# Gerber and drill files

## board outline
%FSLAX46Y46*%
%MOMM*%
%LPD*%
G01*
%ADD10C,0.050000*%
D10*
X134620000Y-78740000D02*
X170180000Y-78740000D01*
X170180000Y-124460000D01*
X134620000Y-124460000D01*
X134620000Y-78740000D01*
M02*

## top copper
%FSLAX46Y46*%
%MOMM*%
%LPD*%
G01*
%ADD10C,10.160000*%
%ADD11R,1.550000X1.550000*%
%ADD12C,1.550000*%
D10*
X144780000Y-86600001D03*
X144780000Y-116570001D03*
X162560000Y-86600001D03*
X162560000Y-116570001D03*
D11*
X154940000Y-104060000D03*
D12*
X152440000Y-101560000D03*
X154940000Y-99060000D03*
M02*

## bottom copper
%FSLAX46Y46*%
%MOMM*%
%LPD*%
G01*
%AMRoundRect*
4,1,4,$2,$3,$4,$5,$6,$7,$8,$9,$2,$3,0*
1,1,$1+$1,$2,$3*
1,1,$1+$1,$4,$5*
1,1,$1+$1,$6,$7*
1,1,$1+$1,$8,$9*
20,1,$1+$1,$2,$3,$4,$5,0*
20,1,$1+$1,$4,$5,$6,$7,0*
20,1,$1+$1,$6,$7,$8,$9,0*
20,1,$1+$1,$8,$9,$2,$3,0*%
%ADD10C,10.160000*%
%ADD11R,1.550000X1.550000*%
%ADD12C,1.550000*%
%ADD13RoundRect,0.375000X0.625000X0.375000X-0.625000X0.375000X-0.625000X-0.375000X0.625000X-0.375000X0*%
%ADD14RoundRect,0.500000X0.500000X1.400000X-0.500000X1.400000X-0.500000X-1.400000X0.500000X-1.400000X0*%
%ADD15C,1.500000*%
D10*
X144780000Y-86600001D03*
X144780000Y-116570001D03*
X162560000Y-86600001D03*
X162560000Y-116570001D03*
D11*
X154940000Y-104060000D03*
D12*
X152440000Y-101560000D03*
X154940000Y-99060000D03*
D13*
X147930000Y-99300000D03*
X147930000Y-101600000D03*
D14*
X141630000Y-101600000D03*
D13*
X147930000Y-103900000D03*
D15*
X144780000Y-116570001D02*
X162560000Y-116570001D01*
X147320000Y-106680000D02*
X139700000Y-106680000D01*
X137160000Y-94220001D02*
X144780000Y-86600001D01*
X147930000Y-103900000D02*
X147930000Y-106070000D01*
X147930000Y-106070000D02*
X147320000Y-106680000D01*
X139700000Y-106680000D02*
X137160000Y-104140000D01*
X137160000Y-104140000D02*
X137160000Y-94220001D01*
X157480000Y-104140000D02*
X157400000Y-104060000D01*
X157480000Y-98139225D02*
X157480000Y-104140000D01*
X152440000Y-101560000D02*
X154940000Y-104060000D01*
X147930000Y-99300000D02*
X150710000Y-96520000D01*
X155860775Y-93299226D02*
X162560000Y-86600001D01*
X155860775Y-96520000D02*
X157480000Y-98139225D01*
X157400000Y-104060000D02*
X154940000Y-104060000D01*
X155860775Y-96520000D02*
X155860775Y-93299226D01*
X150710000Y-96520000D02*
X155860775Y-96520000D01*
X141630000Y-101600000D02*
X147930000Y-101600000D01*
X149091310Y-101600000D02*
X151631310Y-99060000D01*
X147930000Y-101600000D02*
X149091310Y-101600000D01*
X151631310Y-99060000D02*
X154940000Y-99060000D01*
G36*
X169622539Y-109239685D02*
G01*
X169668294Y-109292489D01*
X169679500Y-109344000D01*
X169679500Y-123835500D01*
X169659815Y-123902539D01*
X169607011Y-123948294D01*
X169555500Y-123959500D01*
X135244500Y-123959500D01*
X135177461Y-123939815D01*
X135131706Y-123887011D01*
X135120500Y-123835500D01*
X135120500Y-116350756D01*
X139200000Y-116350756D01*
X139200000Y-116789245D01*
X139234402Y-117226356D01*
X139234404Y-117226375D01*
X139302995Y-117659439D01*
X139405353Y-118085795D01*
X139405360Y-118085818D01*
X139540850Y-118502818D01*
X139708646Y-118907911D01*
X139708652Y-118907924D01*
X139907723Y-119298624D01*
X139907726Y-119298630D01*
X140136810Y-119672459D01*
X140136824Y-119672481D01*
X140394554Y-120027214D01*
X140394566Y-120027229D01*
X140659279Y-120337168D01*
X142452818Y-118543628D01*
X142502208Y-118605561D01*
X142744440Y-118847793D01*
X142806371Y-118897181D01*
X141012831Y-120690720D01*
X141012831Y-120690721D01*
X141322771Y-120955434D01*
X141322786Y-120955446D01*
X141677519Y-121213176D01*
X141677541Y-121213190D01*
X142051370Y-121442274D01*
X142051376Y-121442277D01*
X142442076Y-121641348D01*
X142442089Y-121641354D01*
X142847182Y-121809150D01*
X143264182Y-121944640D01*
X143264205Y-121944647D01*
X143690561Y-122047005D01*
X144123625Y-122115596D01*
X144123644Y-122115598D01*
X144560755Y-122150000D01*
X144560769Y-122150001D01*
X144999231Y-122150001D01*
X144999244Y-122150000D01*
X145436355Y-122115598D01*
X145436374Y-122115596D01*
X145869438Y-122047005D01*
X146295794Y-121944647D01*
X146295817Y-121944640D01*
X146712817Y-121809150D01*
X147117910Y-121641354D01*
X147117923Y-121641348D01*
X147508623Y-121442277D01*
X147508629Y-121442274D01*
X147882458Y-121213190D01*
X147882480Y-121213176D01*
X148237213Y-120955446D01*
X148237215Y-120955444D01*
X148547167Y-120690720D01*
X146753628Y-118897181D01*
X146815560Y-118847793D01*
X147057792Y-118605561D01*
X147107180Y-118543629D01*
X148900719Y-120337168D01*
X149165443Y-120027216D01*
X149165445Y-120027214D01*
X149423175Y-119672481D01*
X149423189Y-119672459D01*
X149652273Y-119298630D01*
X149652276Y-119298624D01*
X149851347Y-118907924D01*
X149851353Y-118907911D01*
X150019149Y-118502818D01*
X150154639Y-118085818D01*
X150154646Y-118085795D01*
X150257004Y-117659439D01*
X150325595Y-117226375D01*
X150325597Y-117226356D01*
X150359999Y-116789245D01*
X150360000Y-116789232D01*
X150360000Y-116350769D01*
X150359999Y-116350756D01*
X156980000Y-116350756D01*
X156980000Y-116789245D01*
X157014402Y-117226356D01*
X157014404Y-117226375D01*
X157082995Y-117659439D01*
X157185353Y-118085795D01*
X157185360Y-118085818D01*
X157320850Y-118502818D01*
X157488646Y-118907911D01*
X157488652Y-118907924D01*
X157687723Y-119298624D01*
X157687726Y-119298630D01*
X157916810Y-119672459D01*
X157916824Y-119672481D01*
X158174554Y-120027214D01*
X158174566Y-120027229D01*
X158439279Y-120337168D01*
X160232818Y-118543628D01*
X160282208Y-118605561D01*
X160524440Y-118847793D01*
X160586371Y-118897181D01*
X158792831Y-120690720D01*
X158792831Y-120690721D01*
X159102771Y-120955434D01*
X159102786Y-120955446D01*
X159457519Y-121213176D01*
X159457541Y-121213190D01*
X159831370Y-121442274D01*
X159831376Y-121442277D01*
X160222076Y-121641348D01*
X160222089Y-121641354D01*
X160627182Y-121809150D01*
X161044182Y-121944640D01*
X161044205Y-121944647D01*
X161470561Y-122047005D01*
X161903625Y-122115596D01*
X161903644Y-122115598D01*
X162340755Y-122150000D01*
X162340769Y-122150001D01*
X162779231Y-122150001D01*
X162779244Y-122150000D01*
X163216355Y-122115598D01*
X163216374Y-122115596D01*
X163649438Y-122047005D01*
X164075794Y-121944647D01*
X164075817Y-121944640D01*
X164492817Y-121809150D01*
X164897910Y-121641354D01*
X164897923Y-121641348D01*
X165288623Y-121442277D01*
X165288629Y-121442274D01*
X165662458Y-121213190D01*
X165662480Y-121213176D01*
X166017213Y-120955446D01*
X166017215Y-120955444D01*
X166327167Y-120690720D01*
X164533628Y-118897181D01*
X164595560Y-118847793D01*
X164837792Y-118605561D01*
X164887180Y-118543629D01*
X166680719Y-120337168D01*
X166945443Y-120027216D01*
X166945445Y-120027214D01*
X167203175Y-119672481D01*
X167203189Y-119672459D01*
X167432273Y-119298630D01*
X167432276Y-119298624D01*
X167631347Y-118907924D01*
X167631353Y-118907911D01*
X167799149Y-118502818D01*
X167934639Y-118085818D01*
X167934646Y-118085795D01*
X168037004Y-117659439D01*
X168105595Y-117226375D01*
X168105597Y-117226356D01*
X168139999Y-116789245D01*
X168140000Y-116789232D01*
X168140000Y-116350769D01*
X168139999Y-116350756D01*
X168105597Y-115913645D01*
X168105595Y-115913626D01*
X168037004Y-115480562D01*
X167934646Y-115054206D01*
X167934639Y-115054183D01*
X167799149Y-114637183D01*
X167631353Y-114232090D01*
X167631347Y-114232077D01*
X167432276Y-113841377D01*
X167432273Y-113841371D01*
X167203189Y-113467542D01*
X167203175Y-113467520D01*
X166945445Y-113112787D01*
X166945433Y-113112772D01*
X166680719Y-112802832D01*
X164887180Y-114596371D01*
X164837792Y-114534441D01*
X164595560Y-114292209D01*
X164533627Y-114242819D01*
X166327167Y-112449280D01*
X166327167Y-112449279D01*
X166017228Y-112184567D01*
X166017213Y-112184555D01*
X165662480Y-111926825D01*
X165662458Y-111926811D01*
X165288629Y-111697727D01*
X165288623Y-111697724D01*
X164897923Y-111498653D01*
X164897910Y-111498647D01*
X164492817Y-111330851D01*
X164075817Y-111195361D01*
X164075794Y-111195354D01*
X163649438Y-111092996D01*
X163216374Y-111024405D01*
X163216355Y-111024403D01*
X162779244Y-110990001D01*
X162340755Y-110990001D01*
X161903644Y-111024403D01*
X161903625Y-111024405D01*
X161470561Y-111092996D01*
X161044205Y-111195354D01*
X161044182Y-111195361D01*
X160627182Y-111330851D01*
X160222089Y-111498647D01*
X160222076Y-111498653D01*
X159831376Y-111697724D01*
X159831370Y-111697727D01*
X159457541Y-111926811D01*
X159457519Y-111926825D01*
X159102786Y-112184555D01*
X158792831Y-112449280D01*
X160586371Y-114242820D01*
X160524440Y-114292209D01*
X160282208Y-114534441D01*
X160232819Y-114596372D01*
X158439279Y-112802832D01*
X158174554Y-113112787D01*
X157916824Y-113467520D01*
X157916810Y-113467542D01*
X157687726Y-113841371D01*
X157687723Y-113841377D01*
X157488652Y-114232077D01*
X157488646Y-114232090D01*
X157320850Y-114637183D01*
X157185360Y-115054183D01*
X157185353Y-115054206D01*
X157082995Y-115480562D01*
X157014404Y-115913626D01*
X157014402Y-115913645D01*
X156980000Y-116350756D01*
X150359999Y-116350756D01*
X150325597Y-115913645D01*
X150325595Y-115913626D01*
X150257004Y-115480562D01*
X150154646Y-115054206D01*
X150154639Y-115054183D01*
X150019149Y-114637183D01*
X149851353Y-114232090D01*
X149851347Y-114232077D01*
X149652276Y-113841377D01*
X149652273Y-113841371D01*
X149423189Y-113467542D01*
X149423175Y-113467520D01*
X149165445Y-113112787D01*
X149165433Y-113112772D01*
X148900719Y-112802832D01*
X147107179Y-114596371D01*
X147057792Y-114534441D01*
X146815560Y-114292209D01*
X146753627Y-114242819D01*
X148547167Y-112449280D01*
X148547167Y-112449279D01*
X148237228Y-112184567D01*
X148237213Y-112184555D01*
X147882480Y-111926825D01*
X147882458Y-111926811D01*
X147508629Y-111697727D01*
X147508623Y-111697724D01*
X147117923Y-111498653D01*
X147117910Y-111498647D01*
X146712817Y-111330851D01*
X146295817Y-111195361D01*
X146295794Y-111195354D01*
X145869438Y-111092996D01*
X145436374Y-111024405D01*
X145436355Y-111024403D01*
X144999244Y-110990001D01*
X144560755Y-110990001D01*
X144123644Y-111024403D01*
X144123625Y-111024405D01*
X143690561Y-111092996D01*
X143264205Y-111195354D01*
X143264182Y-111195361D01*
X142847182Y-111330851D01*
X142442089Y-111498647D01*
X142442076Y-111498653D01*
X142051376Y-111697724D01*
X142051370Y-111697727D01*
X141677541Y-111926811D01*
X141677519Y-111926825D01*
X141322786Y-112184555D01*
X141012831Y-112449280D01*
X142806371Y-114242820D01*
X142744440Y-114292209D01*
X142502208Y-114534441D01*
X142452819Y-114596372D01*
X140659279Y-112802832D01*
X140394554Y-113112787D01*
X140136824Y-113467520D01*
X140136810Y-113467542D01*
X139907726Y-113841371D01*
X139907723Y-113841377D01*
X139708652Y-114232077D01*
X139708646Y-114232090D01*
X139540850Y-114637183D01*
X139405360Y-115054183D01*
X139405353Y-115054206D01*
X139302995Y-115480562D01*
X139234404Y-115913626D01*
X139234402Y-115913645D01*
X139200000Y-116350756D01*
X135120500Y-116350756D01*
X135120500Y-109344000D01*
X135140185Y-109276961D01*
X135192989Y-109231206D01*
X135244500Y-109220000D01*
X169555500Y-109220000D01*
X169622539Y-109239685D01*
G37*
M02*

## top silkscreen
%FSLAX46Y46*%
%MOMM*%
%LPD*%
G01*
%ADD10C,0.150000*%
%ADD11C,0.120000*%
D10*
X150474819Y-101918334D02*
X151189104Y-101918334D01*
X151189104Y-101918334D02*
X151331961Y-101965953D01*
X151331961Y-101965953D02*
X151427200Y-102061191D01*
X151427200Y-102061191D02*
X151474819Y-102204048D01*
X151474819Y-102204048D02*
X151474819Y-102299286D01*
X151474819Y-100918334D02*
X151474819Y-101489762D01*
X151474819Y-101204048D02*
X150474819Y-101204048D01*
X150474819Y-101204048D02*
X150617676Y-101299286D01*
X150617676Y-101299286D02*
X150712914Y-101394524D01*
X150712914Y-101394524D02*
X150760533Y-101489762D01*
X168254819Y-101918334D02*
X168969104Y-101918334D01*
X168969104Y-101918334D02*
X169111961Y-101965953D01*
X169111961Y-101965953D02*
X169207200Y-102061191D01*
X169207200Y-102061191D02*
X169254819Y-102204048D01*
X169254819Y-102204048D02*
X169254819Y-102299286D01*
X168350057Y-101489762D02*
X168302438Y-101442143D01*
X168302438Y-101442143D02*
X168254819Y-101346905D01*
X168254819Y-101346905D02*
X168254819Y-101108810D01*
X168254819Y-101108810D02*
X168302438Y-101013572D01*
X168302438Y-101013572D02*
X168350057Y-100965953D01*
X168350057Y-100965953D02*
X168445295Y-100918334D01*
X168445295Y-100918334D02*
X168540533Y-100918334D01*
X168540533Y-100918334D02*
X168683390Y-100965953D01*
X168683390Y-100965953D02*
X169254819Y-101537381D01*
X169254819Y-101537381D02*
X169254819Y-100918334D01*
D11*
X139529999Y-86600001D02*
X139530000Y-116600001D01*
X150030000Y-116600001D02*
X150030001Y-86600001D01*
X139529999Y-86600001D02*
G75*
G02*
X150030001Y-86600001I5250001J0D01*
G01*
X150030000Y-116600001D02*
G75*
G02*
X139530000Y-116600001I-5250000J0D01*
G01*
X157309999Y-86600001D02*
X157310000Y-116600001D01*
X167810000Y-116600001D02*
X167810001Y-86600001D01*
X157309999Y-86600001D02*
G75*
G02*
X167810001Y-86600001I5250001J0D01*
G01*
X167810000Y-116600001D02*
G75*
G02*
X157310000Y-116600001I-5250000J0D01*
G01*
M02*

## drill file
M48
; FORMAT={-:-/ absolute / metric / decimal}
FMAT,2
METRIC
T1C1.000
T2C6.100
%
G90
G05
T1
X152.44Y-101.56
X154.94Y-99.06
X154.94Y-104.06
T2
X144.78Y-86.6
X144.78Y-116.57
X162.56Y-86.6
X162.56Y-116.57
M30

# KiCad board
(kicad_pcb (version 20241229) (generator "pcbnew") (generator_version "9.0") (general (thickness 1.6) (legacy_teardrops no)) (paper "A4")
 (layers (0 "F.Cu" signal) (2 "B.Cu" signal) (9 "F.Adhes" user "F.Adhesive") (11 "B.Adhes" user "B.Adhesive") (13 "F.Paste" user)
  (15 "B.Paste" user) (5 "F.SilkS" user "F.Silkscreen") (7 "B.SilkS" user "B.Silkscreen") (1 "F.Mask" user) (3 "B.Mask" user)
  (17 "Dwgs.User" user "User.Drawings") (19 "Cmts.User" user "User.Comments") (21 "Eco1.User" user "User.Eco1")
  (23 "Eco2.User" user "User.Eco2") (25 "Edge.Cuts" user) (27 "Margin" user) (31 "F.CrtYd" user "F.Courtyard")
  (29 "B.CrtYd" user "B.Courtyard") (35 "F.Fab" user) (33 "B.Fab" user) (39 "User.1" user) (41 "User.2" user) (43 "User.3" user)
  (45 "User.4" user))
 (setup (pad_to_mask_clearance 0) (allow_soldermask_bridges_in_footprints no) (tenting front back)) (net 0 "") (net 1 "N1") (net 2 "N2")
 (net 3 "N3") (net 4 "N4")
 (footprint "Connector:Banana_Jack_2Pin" (layer "F.Cu") (at 144.78 86.600001 -90)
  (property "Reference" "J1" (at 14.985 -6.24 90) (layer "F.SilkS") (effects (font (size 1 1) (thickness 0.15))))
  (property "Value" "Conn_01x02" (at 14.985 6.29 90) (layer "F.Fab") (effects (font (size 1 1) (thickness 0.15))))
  (fp_line (start 0 5.250001) (end 30 5.25) (stroke (width 0.12) (type solid)) (layer "F.SilkS"))
  (fp_line (start 30 -5.25) (end 0 -5.250001) (stroke (width 0.12) (type solid)) (layer "F.SilkS"))
  (fp_arc (start 0 5.250001) (mid -5.250001 0) (end 0 -5.250001) (stroke (width 0.12) (type solid)) (layer "F.SilkS"))
  (fp_arc (start 30 -5.25) (mid 35.25 0) (end 30 5.25) (stroke (width 0.12) (type solid)) (layer "F.SilkS"))
  (pad "1" thru_hole circle (at 0 0 270) (size 10.16 10.16) (drill 6.1) (layers "*.Cu" "*.Mask") (remove_unused_layers no) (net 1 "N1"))
  (pad "2" thru_hole circle (at 29.97 0 270) (size 10.16 10.16) (drill 6.1) (layers "*.Cu" "*.Mask") (remove_unused_layers no) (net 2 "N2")))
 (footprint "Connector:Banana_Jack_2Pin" (layer "F.Cu") (at 162.56 86.600001 -90)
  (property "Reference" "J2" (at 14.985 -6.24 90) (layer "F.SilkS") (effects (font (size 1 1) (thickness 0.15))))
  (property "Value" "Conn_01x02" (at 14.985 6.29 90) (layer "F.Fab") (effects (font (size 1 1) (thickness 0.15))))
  (fp_line (start 0 5.250001) (end 30 5.25) (stroke (width 0.12) (type solid)) (layer "F.SilkS"))
  (fp_line (start 30 -5.25) (end 0 -5.250001) (stroke (width 0.12) (type solid)) (layer "F.SilkS"))
  (fp_arc (start 0 5.250001) (mid -5.250001 0) (end 0 -5.250001) (stroke (width 0.12) (type solid)) (layer "F.SilkS"))
  (fp_arc (start 30 -5.25) (mid 35.25 0) (end 30 5.25) (stroke (width 0.12) (type solid)) (layer "F.SilkS"))
  (pad "1" thru_hole circle (at 0 0 270) (size 10.16 10.16) (drill 6.1) (layers "*.Cu" "*.Mask") (remove_unused_layers no) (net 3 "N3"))
  (pad "2" thru_hole circle (at 29.97 0 270) (size 10.16 10.16) (drill 6.1) (layers "*.Cu" "*.Mask") (remove_unused_layers no) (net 2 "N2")))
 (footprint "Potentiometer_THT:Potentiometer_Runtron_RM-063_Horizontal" (layer "B.Cu") (at 154.94 104.06 90)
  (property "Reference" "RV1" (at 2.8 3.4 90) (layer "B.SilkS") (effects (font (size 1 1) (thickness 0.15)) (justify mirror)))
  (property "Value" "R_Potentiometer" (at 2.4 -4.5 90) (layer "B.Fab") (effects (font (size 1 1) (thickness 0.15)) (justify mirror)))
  (pad "1" thru_hole rect (at 0 0 90) (size 1.55 1.55) (drill 1) (layers "*.Cu" "*.Mask") (remove_unused_layers no) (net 3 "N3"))
  (pad "2" thru_hole circle (at 2.5 -2.5 90) (size 1.55 1.55) (drill 1) (layers "*.Cu" "*.Mask") (remove_unused_layers no) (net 3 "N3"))
  (pad "3" thru_hole circle (at 5 0 90) (size 1.55 1.55) (drill 1) (layers "*.Cu" "*.Mask") (remove_unused_layers no) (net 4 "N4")))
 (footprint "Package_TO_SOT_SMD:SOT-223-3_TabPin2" (layer "B.Cu") (at 144.78 101.6 180)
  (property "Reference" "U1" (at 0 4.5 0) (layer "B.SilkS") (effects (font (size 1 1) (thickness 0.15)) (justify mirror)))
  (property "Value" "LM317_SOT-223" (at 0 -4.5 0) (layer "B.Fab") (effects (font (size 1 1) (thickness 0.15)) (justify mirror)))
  (pad "1" smd roundrect (at -3.15 2.3 180) (size 2 1.5) (layers "B.Cu" "B.Mask" "B.Paste") (roundrect_rratio 0.25) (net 3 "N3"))
  (pad "2" smd roundrect (at -3.15 0 180) (size 2 1.5) (layers "B.Cu" "B.Mask" "B.Paste") (roundrect_rratio 0.25) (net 4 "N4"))
  (pad "2" smd roundrect (at 3.15 0 180) (size 2 3.8) (layers "B.Cu" "B.Mask" "B.Paste") (roundrect_rratio 0.25) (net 4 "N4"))
  (pad "3" smd roundrect (at -3.15 -2.3 180) (size 2 1.5) (layers "B.Cu" "B.Mask" "B.Paste") (roundrect_rratio 0.25) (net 1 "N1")))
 (gr_rect (start 134.62 78.74) (end 170.18 124.46) (stroke (width 0.05) (type default)) (fill no) (layer "Edge.Cuts"))
 (segment (start 144.78 116.570001) (end 162.56 116.570001) (width 1.5) (layer "B.Cu") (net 2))
 (segment (start 147.32 106.68) (end 139.7 106.68) (width 1.5) (layer "B.Cu") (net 1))
 (segment (start 137.16 94.220001) (end 144.78 86.600001) (width 1.5) (layer "B.Cu") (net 1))
 (segment (start 147.93 103.9) (end 147.93 106.07) (width 1.5) (layer "B.Cu") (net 1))
 (segment (start 147.93 106.07) (end 147.32 106.68) (width 1.5) (layer "B.Cu") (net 1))
 (segment (start 139.7 106.68) (end 137.16 104.14) (width 1.5) (layer "B.Cu") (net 1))
 (segment (start 137.16 104.14) (end 137.16 94.220001) (width 1.5) (layer "B.Cu") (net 1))
 (segment (start 157.48 104.14) (end 157.4 104.06) (width 1.5) (layer "B.Cu") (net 3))
 (segment (start 157.48 98.139225) (end 157.48 104.14) (width 1.5) (layer "B.Cu") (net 3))
 (segment (start 152.44 101.56) (end 154.94 104.06) (width 1.5) (layer "B.Cu") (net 3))
 (segment (start 147.93 99.3) (end 150.71 96.52) (width 1.5) (layer "B.Cu") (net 3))
 (segment (start 155.860775 93.299226) (end 162.56 86.600001) (width 1.5) (layer "B.Cu") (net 3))
 (segment (start 155.860775 96.52) (end 157.48 98.139225) (width 1.5) (layer "B.Cu") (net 3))
 (segment (start 157.4 104.06) (end 154.94 104.06) (width 1.5) (layer "B.Cu") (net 3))
 (segment (start 155.860775 96.52) (end 155.860775 93.299226) (width 1.5) (layer "B.Cu") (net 3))
 (segment (start 150.71 96.52) (end 155.860775 96.52) (width 1.5) (layer "B.Cu") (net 3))
 (segment (start 141.63 101.6) (end 147.93 101.6) (width 1.5) (layer "B.Cu") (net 4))
 (segment (start 149.09131 101.6) (end 151.63131 99.06) (width 1.5) (layer "B.Cu") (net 4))
 (segment (start 147.93 101.6) (end 149.09131 101.6) (width 1.5) (layer "B.Cu") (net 4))
 (segment (start 151.63131 99.06) (end 154.94 99.06) (width 1.5) (layer "B.Cu") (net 4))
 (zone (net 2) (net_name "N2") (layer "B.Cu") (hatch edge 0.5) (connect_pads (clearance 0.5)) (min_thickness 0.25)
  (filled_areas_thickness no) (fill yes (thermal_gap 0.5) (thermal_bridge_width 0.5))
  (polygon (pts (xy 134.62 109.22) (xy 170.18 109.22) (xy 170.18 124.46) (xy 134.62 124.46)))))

